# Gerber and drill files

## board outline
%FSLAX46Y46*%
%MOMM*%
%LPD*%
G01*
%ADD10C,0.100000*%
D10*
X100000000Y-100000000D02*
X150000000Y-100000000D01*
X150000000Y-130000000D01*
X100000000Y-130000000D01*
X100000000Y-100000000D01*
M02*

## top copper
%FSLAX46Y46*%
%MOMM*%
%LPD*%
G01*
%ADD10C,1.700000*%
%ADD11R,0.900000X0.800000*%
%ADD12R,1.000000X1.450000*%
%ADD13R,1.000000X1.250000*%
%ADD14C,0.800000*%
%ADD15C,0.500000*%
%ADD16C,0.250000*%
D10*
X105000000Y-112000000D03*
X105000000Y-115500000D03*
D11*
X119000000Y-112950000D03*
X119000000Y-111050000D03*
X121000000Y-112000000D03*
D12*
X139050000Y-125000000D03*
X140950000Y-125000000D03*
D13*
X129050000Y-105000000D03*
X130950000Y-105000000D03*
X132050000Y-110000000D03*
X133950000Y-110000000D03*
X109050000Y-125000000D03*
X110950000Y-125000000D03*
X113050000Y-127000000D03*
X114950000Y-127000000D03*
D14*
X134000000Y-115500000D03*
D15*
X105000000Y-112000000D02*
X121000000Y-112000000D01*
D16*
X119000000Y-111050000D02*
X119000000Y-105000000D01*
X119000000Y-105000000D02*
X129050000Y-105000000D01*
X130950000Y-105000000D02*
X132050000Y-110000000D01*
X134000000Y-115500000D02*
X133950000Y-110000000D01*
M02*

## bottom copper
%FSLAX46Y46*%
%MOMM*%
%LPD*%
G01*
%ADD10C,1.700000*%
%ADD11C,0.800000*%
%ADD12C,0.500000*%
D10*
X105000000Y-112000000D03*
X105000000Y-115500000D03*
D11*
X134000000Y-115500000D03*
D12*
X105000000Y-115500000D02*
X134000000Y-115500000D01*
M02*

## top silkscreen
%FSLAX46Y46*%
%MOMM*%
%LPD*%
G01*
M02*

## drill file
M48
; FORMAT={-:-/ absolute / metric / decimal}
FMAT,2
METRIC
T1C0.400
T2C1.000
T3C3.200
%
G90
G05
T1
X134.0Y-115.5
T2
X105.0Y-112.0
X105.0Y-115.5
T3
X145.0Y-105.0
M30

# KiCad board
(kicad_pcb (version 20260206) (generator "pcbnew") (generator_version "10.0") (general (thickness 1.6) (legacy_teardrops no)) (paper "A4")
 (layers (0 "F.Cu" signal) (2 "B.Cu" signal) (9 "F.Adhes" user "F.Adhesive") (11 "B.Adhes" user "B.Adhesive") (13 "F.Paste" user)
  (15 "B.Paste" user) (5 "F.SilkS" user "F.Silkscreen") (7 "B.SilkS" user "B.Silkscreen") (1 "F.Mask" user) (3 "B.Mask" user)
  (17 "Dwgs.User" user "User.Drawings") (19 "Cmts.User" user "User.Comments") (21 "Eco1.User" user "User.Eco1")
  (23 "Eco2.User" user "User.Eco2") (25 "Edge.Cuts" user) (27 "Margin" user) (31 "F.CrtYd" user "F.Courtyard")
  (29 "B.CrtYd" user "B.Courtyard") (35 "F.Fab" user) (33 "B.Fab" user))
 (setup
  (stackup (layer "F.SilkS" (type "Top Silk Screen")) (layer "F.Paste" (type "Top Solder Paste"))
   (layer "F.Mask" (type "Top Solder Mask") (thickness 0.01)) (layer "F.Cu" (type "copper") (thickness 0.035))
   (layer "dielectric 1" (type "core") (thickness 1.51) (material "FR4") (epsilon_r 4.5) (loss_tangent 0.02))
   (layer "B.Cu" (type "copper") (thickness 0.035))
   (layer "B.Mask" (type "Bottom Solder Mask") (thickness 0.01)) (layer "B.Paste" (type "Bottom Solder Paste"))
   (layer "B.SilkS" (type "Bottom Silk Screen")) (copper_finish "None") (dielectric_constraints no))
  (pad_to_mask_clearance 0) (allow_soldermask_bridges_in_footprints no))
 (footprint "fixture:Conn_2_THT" (layer "F.Cu") (at 105 112)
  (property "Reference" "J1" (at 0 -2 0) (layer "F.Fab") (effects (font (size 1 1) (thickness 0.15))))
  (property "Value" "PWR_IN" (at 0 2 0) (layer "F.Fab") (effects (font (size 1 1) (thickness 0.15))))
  (pad "1" thru_hole circle (at 0 0) (size 1.7 1.7) (drill 1) (layers "*.Cu" "*.Mask") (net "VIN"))
  (pad "2" thru_hole circle (at 0 3.5) (size 1.7 1.7) (drill 1) (layers "*.Cu" "*.Mask") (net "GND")))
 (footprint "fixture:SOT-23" (layer "F.Cu") (at 120 112)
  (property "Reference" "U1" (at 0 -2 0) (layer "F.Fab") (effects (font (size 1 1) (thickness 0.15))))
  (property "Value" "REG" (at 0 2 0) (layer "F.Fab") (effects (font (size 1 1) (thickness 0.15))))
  (pad "1" smd rect (at -1 0.95) (size 0.9 0.8) (layers "F.Cu" "F.Paste" "F.Mask") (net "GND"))
  (pad "2" smd rect (at -1 -0.95) (size 0.9 0.8) (layers "F.Cu" "F.Paste" "F.Mask") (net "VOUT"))
  (pad "3" smd rect (at 1 0) (size 0.9 0.8) (layers "F.Cu" "F.Paste" "F.Mask") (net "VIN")))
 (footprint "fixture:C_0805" (layer "F.Cu") (at 140 125)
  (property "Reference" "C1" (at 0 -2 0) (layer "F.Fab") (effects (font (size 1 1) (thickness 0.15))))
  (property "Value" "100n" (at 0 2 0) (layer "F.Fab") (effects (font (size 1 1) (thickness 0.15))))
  (pad "1" smd rect (at -0.95 0) (size 1 1.45) (layers "F.Cu" "F.Paste" "F.Mask") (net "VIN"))
  (pad "2" smd rect (at 0.95 0) (size 1 1.45) (layers "F.Cu" "F.Paste" "F.Mask") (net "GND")))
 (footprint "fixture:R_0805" (layer "F.Cu") (at 130 105)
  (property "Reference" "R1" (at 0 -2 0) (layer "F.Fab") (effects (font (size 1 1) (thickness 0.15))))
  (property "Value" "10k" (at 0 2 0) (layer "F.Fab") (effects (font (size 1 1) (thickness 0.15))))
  (pad "1" smd rect (at -0.95 0) (size 1 1.25) (layers "F.Cu" "F.Paste" "F.Mask") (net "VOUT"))
  (pad "2" smd rect (at 0.95 0) (size 1 1.25) (layers "F.Cu" "F.Paste" "F.Mask") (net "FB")))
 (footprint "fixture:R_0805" (layer "F.Cu") (at 133 110)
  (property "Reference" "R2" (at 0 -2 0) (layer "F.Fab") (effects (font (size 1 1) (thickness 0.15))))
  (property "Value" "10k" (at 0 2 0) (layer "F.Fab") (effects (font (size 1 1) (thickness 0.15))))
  (pad "1" smd rect (at -0.95 0) (size 1 1.25) (layers "F.Cu" "F.Paste" "F.Mask") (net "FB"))
  (pad "2" smd rect (at 0.95 0) (size 1 1.25) (layers "F.Cu" "F.Paste" "F.Mask") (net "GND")))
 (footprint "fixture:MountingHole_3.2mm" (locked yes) (layer "F.Cu") (at 145 105)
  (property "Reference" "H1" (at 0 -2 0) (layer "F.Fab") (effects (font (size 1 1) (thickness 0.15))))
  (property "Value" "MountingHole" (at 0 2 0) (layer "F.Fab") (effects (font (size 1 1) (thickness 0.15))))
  (pad "" np_thru_hole circle (at 0 0) (size 3.2 3.2) (drill 3.2) (layers "*.Cu" "*.Mask")))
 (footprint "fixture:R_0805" (layer "F.Cu") (at 110 125)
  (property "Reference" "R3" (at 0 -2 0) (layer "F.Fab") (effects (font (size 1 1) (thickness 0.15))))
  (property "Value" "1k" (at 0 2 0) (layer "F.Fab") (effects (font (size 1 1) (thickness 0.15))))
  (pad "1" smd rect (at -0.95 0) (size 1 1.25) (layers "F.Cu" "F.Paste" "F.Mask") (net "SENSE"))
  (pad "2" smd rect (at 0.95 0) (size 1 1.25) (layers "F.Cu" "F.Paste" "F.Mask")))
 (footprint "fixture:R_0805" (layer "F.Cu") (at 114 127)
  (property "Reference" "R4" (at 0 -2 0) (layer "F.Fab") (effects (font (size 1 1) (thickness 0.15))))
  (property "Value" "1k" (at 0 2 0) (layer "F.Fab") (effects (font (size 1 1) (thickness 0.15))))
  (pad "1" smd rect (at -0.95 0) (size 1 1.25) (layers "F.Cu" "F.Paste" "F.Mask") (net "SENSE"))
  (pad "2" smd rect (at 0.95 0) (size 1 1.25) (layers "F.Cu" "F.Paste" "F.Mask")))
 (gr_rect (start 100 100) (end 150 130) (stroke (width 0.1) (type solid)) (fill no) (layer "Edge.Cuts"))
 (segment (start 105 112) (end 121 112) (width 0.5) (layer "F.Cu") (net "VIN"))
 (segment (start 119 111.05) (end 119 105) (width 0.25) (layer "F.Cu") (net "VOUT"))
 (segment (start 119 105) (end 129.05 105) (width 0.25) (layer "F.Cu") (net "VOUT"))
 (segment (start 130.95 105) (end 132.05 110) (width 0.25) (layer "F.Cu") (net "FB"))
 (segment (start 105 115.5) (end 134 115.5) (width 0.5) (layer "B.Cu") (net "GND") (locked yes))
 (segment (start 134 115.5) (end 133.95 110) (width 0.25) (layer "F.Cu") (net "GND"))
 (via (at 134 115.5) (size 0.8) (drill 0.4) (layers "F.Cu" "B.Cu") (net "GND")))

